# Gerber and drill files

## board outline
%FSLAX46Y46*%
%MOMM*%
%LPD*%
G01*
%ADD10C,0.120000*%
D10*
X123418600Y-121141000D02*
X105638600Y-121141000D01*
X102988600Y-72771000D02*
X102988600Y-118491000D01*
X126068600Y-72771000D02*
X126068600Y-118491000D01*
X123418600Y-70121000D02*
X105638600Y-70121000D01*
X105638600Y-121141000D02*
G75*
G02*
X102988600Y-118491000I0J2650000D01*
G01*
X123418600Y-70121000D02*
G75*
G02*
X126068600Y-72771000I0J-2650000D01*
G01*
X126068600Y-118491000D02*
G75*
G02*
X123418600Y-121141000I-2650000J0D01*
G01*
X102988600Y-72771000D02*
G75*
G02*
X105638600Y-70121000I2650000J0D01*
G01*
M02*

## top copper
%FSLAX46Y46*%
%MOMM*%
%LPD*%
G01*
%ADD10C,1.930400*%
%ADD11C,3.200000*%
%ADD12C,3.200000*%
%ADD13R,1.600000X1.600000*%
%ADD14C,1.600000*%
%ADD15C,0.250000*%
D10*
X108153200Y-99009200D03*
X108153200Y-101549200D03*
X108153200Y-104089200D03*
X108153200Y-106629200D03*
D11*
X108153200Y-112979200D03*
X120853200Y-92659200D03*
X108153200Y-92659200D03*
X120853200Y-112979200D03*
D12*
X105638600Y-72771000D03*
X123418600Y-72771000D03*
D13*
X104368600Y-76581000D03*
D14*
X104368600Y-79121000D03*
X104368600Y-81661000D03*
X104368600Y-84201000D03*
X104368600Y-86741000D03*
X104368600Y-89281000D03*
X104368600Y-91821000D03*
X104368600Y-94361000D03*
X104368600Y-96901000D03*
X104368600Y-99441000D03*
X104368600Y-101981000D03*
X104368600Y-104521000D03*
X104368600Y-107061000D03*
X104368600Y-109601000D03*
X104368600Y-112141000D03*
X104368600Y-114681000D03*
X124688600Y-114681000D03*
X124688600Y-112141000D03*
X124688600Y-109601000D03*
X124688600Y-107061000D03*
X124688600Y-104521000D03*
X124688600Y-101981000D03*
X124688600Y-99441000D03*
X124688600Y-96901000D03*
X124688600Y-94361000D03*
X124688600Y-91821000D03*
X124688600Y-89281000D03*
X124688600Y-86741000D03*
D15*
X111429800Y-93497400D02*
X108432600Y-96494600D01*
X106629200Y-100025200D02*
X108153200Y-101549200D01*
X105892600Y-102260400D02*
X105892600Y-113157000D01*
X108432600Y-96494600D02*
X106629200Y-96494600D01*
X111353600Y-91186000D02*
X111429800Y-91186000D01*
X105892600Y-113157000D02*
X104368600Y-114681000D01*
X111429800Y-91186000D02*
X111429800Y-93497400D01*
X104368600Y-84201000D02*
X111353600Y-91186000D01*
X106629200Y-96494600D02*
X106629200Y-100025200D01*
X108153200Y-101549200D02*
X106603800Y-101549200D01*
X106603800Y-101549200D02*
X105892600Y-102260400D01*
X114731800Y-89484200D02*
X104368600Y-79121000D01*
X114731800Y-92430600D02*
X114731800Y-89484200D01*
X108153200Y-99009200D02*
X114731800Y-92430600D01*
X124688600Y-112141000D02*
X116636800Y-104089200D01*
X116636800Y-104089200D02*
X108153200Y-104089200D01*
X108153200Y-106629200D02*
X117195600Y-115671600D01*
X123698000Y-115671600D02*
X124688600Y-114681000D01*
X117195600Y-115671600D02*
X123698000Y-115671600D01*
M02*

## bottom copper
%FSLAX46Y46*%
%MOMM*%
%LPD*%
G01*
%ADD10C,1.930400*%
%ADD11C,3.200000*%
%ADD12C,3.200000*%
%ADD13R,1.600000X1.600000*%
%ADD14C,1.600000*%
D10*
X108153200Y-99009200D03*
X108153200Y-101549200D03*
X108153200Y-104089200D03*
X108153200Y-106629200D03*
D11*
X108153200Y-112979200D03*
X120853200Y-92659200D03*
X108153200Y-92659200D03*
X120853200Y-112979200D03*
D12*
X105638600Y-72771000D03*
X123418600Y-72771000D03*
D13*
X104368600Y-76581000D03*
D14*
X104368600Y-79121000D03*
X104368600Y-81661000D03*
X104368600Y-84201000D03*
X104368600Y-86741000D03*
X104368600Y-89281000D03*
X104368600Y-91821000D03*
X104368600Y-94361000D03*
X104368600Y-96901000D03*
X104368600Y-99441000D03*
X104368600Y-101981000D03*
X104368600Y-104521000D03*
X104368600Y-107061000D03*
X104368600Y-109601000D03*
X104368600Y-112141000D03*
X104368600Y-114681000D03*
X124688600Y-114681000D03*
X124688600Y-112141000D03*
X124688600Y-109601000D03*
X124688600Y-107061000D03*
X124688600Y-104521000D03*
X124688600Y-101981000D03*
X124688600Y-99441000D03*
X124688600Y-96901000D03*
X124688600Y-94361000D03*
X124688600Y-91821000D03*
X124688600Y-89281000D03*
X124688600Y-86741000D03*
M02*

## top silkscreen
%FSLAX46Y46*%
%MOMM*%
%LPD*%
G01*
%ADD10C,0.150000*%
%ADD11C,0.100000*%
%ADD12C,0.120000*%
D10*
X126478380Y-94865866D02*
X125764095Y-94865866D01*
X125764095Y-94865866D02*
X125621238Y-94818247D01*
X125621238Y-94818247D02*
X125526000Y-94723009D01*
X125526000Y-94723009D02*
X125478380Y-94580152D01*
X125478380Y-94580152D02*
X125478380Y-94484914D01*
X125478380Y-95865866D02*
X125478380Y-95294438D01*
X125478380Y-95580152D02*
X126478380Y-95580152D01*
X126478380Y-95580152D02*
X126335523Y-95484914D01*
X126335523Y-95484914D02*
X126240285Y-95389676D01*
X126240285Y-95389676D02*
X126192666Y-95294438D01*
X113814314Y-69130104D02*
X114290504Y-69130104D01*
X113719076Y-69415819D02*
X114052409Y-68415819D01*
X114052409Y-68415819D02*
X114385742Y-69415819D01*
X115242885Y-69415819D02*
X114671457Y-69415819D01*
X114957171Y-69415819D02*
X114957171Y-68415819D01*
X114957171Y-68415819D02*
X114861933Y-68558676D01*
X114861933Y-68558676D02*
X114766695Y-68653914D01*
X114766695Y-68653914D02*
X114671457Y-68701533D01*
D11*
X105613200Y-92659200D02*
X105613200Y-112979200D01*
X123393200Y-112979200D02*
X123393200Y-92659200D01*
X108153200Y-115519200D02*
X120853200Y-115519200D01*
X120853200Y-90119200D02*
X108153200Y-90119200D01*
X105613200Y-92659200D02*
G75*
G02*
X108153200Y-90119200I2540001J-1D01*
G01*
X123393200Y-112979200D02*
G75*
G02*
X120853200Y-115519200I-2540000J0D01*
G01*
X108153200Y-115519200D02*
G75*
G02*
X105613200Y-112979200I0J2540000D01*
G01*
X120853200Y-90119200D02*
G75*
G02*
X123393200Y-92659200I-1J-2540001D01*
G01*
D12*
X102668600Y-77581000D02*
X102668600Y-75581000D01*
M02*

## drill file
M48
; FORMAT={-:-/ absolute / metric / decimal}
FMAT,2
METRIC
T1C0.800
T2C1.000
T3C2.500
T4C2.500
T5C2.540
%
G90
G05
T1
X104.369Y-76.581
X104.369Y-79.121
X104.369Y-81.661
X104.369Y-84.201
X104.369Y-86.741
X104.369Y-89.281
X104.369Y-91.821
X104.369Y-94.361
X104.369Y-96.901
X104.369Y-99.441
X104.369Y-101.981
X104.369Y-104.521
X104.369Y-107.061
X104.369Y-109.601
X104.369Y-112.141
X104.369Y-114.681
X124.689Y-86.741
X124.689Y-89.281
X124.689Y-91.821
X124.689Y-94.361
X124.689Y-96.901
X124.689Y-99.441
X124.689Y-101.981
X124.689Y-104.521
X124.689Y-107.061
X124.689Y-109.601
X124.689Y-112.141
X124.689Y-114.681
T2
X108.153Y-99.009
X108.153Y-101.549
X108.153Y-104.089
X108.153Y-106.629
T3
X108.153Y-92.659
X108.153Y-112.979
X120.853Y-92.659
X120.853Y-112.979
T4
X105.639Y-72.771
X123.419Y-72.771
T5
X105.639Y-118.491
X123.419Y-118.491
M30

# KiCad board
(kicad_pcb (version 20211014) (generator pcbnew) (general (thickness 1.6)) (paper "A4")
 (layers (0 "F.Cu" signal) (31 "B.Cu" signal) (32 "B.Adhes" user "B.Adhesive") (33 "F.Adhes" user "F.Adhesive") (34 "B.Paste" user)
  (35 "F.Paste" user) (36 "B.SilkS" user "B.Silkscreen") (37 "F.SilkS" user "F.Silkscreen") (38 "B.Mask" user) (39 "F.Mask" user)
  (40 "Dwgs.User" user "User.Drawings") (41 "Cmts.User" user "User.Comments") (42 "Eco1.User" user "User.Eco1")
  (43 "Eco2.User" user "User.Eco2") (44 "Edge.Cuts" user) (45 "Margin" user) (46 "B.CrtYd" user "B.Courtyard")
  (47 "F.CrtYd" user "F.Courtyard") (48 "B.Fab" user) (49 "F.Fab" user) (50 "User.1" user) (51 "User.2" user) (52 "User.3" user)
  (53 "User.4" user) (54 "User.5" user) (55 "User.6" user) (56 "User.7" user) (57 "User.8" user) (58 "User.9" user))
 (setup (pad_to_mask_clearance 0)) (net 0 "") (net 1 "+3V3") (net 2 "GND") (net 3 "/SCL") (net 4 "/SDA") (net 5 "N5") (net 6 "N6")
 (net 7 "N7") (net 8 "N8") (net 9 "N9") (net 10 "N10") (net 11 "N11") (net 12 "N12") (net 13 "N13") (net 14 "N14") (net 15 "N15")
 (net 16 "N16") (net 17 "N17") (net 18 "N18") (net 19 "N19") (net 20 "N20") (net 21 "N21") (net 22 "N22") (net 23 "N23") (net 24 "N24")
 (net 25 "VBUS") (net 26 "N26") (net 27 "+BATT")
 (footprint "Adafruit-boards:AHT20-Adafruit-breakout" (layer "F.Cu") (at 113.2332 102.8192 -90)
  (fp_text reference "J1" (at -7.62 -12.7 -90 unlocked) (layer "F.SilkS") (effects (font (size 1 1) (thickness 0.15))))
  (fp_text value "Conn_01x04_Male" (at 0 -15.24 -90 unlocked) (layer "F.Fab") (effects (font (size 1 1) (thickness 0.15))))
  (fp_line (start -10.16 7.62) (end 10.16 7.62) (layer "F.SilkS") (width 0.1))
  (fp_line (start 10.16 -10.16) (end -10.16 -10.16) (layer "F.SilkS") (width 0.1))
  (fp_line (start 12.7 5.08) (end 12.7 -7.62) (layer "F.SilkS") (width 0.1))
  (fp_line (start -12.7 -7.62) (end -12.7 5.08) (layer "F.SilkS") (width 0.1))
  (fp_arc (start -10.16 7.62) (mid -11.956051 6.876051) (end -12.7 5.08) (layer "F.SilkS") (width 0.1))
  (fp_arc (start 10.16 -10.16) (mid 11.956051 -9.416051) (end 12.7 -7.62) (layer "F.SilkS") (width 0.1))
  (fp_arc (start 12.7 5.08) (mid 11.956051 6.876051) (end 10.16 7.62) (layer "F.SilkS") (width 0.1))
  (fp_arc (start -12.7 -7.62) (mid -11.956051 -9.416051) (end -10.16 -10.16) (layer "F.SilkS") (width 0.1))
  (pad "1" thru_hole circle (at -3.81 5.08) (size 1.9304 1.9304) (drill 1) (layers *.Cu *.Mask) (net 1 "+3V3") (solder_mask_margin 0.0508))
  (pad "2" thru_hole circle (at -1.27 5.08) (size 1.9304 1.9304) (drill 1) (layers *.Cu *.Mask) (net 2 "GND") (solder_mask_margin 0.0508))
  (pad "3" thru_hole circle (at 1.27 5.08) (size 1.9304 1.9304) (drill 1) (layers *.Cu *.Mask) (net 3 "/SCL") (solder_mask_margin 0.0508))
  (pad "4" thru_hole circle (at 3.81 5.08) (size 1.9304 1.9304) (drill 1) (layers *.Cu *.Mask) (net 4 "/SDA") (solder_mask_margin 0.0508))
  (pad "P$1" thru_hole circle (at 10.16 5.08 270) (size 3.2 3.2) (drill 2.5) (layers *.Cu *.Mask) (solder_mask_margin 0.0508))
  (pad "P$1" thru_hole circle (at -10.16 -7.62 270) (size 3.2 3.2) (drill 2.5) (layers *.Cu *.Mask) (solder_mask_margin 0.0508))
  (pad "P$1" thru_hole circle (at -10.16 5.08 270) (size 3.2 3.2) (drill 2.5) (layers *.Cu *.Mask) (solder_mask_margin 0.0508))
  (pad "P$1" thru_hole circle (at 10.16 -7.62 270) (size 3.2 3.2) (drill 2.5) (layers *.Cu *.Mask) (solder_mask_margin 0.0508)))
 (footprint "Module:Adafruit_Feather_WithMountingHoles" (layer "F.Cu") (at 104.3686 76.581)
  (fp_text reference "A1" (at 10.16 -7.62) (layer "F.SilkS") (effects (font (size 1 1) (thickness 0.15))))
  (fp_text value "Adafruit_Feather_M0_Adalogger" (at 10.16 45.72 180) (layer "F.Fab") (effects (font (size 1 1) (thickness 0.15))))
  (fp_line (start -1.7 1) (end -1.7 -1) (layer "F.SilkS") (width 0.12))
  (fp_line (start 19.05 44.56) (end 1.27 44.56) (layer "Edge.Cuts") (width 0.12))
  (fp_line (start -1.38 -3.81) (end -1.38 41.91) (layer "Edge.Cuts") (width 0.12))
  (fp_line (start 21.7 -3.81) (end 21.7 41.91) (layer "Edge.Cuts") (width 0.12))
  (fp_line (start 19.05 -6.46) (end 1.27 -6.46) (layer "Edge.Cuts") (width 0.12))
  (fp_arc (start 1.27 44.56) (mid -0.603833 43.783833) (end -1.38 41.91) (layer "Edge.Cuts") (width 0.12))
  (fp_arc (start 19.05 -6.46) (mid 20.923833 -5.683833) (end 21.7 -3.81) (layer "Edge.Cuts") (width 0.12))
  (fp_arc (start 21.7 41.91) (mid 20.923833 43.783833) (end 19.05 44.56) (layer "Edge.Cuts") (width 0.12))
  (fp_arc (start -1.38 -3.81) (mid -0.603833 -5.683833) (end 1.27 -6.46) (layer "Edge.Cuts") (width 0.12))
  (pad "" np_thru_hole circle (at 1.27 -3.81 270) (size 3.2 3.2) (drill 2.5) (layers *.Cu *.Mask))
  (pad "" np_thru_hole circle (at 19.05 -3.81 270) (size 3.2 3.2) (drill 2.5) (layers *.Cu *.Mask))
  (pad "" np_thru_hole circle (at 19.05 41.91 270) (size 2.54 2.54) (drill 2.54) (layers *.Cu *.Mask))
  (pad "" np_thru_hole circle (at 1.27 41.91 270) (size 2.54 2.54) (drill 2.54) (layers *.Cu *.Mask))
  (pad "1" thru_hole rect (at 0 0 180) (size 1.6 1.6) (drill 0.8) (layers *.Cu *.Mask) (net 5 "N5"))
  (pad "2" thru_hole circle (at 0 2.54 180) (size 1.6 1.6) (drill 0.8) (layers *.Cu *.Mask) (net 1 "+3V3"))
  (pad "3" thru_hole circle (at 0 5.08 180) (size 1.6 1.6) (drill 0.8) (layers *.Cu *.Mask) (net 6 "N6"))
  (pad "4" thru_hole circle (at 0 7.62 180) (size 1.6 1.6) (drill 0.8) (layers *.Cu *.Mask) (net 2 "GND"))
  (pad "5" thru_hole circle (at 0 10.16 180) (size 1.6 1.6) (drill 0.8) (layers *.Cu *.Mask) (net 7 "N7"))
  (pad "6" thru_hole circle (at 0 12.7 180) (size 1.6 1.6) (drill 0.8) (layers *.Cu *.Mask) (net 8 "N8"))
  (pad "7" thru_hole circle (at 0 15.24 180) (size 1.6 1.6) (drill 0.8) (layers *.Cu *.Mask) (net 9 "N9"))
  (pad "8" thru_hole circle (at 0 17.78 180) (size 1.6 1.6) (drill 0.8) (layers *.Cu *.Mask) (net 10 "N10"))
  (pad "9" thru_hole circle (at 0 20.32 180) (size 1.6 1.6) (drill 0.8) (layers *.Cu *.Mask) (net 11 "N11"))
  (pad "10" thru_hole circle (at 0 22.86 180) (size 1.6 1.6) (drill 0.8) (layers *.Cu *.Mask) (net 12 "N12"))
  (pad "11" thru_hole circle (at 0 25.4 180) (size 1.6 1.6) (drill 0.8) (layers *.Cu *.Mask) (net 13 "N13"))
  (pad "12" thru_hole circle (at 0 27.94 180) (size 1.6 1.6) (drill 0.8) (layers *.Cu *.Mask) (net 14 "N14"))
  (pad "13" thru_hole circle (at 0 30.48 180) (size 1.6 1.6) (drill 0.8) (layers *.Cu *.Mask) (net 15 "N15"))
  (pad "14" thru_hole circle (at 0 33.02 180) (size 1.6 1.6) (drill 0.8) (layers *.Cu *.Mask) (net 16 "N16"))
  (pad "15" thru_hole circle (at 0 35.56 180) (size 1.6 1.6) (drill 0.8) (layers *.Cu *.Mask) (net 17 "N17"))
  (pad "16" thru_hole circle (at 0 38.1 180) (size 1.6 1.6) (drill 0.8) (layers *.Cu *.Mask) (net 2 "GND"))
  (pad "17" thru_hole circle (at 20.32 38.1 180) (size 1.6 1.6) (drill 0.8) (layers *.Cu *.Mask) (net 4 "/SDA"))
  (pad "18" thru_hole circle (at 20.32 35.56 180) (size 1.6 1.6) (drill 0.8) (layers *.Cu *.Mask) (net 3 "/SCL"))
  (pad "19" thru_hole circle (at 20.32 33.02 180) (size 1.6 1.6) (drill 0.8) (layers *.Cu *.Mask) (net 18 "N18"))
  (pad "20" thru_hole circle (at 20.32 30.48 180) (size 1.6 1.6) (drill 0.8) (layers *.Cu *.Mask) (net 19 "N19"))
  (pad "21" thru_hole circle (at 20.32 27.94 180) (size 1.6 1.6) (drill 0.8) (layers *.Cu *.Mask) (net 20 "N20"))
  (pad "22" thru_hole circle (at 20.32 25.4 180) (size 1.6 1.6) (drill 0.8) (layers *.Cu *.Mask) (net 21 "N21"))
  (pad "23" thru_hole circle (at 20.32 22.86 180) (size 1.6 1.6) (drill 0.8) (layers *.Cu *.Mask) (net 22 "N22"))
  (pad "24" thru_hole circle (at 20.32 20.32 180) (size 1.6 1.6) (drill 0.8) (layers *.Cu *.Mask) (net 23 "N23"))
  (pad "25" thru_hole circle (at 20.32 17.78 180) (size 1.6 1.6) (drill 0.8) (layers *.Cu *.Mask) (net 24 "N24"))
  (pad "26" thru_hole circle (at 20.32 15.24 180) (size 1.6 1.6) (drill 0.8) (layers *.Cu *.Mask) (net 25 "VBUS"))
  (pad "27" thru_hole circle (at 20.32 12.7 180) (size 1.6 1.6) (drill 0.8) (layers *.Cu *.Mask) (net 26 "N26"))
  (pad "28" thru_hole circle (at 20.32 10.16 180) (size 1.6 1.6) (drill 0.8) (layers *.Cu *.Mask) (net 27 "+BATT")))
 (segment (start 111.4298 93.4974) (end 108.4326 96.4946) (width 0.25) (layer "F.Cu") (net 2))
 (segment (start 106.6292 100.0252) (end 108.1532 101.5492) (width 0.25) (layer "F.Cu") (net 2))
 (segment (start 105.8926 102.2604) (end 105.8926 113.157) (width 0.25) (layer "F.Cu") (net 2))
 (segment (start 108.4326 96.4946) (end 106.6292 96.4946) (width 0.25) (layer "F.Cu") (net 2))
 (segment (start 111.3536 91.186) (end 111.4298 91.186) (width 0.25) (layer "F.Cu") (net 2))
 (segment (start 105.8926 113.157) (end 104.3686 114.681) (width 0.25) (layer "F.Cu") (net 2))
 (segment (start 111.4298 91.186) (end 111.4298 93.4974) (width 0.25) (layer "F.Cu") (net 2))
 (segment (start 104.3686 84.201) (end 111.3536 91.186) (width 0.25) (layer "F.Cu") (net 2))
 (segment (start 106.6292 96.4946) (end 106.6292 100.0252) (width 0.25) (layer "F.Cu") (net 2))
 (segment (start 108.1532 101.5492) (end 106.6038 101.5492) (width 0.25) (layer "F.Cu") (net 2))
 (segment (start 106.6038 101.5492) (end 105.8926 102.2604) (width 0.25) (layer "F.Cu") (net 2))
 (segment (start 114.7318 89.4842) (end 104.3686 79.121) (width 0.25) (layer "F.Cu") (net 1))
 (segment (start 114.7318 92.4306) (end 114.7318 89.4842) (width 0.25) (layer "F.Cu") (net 1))
 (segment (start 108.1532 99.0092) (end 114.7318 92.4306) (width 0.25) (layer "F.Cu") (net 1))
 (segment (start 124.6886 112.141) (end 116.6368 104.0892) (width 0.25) (layer "F.Cu") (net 3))
 (segment (start 116.6368 104.0892) (end 108.1532 104.0892) (width 0.25) (layer "F.Cu") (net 3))
 (segment (start 108.1532 106.6292) (end 117.1956 115.6716) (width 0.25) (layer "F.Cu") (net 4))
 (segment (start 123.698 115.6716) (end 124.6886 114.681) (width 0.25) (layer "F.Cu") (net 4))
 (segment (start 117.1956 115.6716) (end 123.698 115.6716) (width 0.25) (layer "F.Cu") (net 4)))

